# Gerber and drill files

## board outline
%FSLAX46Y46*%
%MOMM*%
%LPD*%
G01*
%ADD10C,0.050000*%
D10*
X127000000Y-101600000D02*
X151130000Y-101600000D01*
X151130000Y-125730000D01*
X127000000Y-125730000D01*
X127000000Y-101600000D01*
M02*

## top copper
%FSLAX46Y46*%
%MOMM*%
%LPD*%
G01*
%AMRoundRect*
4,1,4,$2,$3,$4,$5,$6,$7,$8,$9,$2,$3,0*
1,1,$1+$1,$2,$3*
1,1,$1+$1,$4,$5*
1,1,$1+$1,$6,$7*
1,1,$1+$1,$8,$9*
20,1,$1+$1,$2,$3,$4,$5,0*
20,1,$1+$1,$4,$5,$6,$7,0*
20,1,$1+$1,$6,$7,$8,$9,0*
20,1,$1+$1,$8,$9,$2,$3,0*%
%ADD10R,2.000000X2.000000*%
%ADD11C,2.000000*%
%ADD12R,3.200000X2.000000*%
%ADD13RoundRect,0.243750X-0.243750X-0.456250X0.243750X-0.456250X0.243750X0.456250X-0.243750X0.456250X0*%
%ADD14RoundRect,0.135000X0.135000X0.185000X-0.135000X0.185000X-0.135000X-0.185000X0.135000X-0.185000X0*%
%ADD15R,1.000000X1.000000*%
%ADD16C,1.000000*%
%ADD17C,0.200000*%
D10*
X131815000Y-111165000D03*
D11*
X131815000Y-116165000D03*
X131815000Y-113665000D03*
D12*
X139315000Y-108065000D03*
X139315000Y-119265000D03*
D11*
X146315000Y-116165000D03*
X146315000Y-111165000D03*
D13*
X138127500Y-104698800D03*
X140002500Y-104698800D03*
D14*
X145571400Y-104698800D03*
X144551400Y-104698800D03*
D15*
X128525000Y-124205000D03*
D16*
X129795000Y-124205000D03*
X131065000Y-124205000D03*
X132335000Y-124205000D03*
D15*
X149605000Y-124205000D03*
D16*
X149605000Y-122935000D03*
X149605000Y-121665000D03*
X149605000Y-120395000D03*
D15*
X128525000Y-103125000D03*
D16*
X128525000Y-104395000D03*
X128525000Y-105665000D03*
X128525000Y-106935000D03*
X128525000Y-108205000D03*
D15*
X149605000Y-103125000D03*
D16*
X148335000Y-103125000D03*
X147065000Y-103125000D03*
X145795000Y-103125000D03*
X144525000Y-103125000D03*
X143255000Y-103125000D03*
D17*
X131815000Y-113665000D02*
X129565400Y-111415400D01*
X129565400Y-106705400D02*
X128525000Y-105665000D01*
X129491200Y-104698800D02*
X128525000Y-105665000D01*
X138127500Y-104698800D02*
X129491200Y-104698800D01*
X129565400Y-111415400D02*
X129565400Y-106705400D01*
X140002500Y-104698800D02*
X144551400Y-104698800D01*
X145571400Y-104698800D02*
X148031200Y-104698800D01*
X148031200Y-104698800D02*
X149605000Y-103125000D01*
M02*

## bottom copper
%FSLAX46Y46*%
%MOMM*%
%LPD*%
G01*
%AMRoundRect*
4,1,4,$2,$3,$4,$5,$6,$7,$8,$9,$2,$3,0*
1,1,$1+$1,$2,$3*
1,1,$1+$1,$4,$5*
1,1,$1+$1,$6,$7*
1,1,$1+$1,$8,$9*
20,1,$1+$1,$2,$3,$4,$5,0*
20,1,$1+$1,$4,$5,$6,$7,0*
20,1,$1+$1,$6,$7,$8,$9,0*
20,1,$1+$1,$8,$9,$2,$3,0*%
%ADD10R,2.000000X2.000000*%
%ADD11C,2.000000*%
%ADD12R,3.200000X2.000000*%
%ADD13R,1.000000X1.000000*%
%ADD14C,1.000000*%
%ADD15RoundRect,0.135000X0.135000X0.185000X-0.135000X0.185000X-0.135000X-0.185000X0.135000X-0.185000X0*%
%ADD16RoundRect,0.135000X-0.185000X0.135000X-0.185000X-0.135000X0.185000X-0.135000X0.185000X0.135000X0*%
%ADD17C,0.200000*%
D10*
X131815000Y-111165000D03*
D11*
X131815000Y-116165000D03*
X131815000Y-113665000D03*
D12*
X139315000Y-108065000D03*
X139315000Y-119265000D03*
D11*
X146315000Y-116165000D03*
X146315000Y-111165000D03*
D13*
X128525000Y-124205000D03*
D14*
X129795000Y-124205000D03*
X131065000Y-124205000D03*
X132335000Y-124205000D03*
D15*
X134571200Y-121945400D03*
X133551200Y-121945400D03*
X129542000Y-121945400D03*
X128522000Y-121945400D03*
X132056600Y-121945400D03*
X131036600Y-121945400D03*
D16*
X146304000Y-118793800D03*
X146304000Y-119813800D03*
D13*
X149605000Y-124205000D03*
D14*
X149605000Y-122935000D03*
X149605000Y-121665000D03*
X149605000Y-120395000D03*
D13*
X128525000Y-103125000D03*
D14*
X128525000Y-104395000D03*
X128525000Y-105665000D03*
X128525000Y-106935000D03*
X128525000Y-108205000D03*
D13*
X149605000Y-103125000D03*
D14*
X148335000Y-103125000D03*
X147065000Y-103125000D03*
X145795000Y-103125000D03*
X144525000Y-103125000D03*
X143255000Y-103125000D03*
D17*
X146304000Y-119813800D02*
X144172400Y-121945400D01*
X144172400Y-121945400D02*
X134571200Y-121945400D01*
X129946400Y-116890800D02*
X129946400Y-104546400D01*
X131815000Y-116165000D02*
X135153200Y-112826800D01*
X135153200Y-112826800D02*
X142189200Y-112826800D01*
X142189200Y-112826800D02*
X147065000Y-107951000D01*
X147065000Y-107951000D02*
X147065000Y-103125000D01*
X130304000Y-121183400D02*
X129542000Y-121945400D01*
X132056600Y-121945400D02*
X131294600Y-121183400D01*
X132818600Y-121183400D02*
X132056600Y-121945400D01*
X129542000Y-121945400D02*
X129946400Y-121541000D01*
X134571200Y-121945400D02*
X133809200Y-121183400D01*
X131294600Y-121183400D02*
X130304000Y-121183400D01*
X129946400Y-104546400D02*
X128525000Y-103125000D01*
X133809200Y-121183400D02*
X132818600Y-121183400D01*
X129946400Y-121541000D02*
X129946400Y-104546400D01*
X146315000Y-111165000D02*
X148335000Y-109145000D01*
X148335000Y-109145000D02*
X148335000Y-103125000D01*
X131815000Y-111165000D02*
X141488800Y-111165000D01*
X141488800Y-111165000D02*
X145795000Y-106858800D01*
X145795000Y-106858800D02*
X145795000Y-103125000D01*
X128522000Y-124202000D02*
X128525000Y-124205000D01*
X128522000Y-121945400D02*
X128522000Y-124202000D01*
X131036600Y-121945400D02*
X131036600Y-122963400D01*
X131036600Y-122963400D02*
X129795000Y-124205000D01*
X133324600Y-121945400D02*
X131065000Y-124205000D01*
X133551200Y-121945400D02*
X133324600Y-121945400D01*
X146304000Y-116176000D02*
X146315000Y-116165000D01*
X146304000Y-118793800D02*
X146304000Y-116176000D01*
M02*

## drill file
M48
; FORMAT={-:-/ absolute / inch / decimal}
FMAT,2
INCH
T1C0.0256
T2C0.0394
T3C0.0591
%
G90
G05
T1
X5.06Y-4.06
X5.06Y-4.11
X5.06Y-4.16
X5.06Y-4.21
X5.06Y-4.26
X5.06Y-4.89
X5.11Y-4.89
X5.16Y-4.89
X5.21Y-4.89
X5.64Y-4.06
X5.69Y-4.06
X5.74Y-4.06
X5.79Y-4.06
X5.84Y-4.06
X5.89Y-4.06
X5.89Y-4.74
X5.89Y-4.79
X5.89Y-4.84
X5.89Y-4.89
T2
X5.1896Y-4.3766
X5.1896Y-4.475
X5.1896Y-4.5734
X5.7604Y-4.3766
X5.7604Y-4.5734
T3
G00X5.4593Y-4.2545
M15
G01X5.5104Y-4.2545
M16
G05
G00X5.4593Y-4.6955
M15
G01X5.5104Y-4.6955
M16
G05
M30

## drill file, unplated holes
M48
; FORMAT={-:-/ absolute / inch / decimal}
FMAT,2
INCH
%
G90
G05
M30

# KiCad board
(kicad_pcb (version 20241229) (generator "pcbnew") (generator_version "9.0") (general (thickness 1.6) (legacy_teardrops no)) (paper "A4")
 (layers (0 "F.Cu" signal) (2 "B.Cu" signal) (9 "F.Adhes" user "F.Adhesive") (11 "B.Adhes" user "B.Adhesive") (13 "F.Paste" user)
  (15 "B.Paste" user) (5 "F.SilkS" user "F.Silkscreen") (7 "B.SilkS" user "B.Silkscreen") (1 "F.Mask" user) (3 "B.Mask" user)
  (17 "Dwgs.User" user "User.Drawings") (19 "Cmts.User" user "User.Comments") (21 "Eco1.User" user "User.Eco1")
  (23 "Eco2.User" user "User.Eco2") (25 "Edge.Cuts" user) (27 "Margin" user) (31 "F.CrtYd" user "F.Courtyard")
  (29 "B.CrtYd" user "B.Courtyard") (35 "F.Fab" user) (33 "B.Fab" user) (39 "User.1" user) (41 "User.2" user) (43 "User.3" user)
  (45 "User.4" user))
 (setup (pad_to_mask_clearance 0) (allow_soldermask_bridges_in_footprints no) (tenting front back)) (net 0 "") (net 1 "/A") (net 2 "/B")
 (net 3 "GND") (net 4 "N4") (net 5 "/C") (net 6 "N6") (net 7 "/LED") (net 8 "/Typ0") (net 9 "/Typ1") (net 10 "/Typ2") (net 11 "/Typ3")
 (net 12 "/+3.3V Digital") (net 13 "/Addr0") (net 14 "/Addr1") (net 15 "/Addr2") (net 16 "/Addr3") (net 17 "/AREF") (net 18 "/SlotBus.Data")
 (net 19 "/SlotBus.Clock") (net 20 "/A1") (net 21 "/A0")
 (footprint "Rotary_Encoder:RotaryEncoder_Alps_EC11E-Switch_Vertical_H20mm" (layer "F.Cu") (at 131.815 111.165)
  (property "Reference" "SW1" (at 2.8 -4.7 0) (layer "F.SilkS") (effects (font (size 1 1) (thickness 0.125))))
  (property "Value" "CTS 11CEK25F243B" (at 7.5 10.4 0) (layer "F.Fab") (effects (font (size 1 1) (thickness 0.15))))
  (pad "A" thru_hole rect (at 0 0) (size 2 2) (drill 1) (layers "*.Cu" "*.Mask") (remove_unused_layers no) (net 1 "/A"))
  (pad "B" thru_hole circle (at 0 5) (size 2 2) (drill 1) (layers "*.Cu" "*.Mask") (remove_unused_layers no) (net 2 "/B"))
  (pad "C" thru_hole circle (at 0 2.5) (size 2 2) (drill 1) (layers "*.Cu" "*.Mask") (remove_unused_layers no) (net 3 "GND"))
  (pad "MP" thru_hole rect (at 7.5 -3.1) (size 3.2 2) (drill oval 2.8 1.5) (layers "*.Cu" "*.Mask") (remove_unused_layers no))
  (pad "MP" thru_hole rect (at 7.5 8.1) (size 3.2 2) (drill oval 2.8 1.5) (layers "*.Cu" "*.Mask") (remove_unused_layers no))
  (pad "S1" thru_hole circle (at 14.5 5) (size 2 2) (drill 1) (layers "*.Cu" "*.Mask") (remove_unused_layers no) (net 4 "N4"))
  (pad "S2" thru_hole circle (at 14.5 0) (size 2 2) (drill 1) (layers "*.Cu" "*.Mask") (remove_unused_layers no) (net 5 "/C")))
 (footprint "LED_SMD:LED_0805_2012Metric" (layer "F.Cu") (at 139.065 104.6988)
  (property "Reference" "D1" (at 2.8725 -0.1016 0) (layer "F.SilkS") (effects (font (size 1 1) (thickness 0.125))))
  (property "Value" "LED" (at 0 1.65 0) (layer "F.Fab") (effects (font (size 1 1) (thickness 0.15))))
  (pad "1" smd roundrect (at -0.9375 0) (size 0.975 1.4) (layers "F.Cu" "F.Mask" "F.Paste") (roundrect_rratio 0.25) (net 3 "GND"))
  (pad "2" smd roundrect (at 0.9375 0) (size 0.975 1.4) (layers "F.Cu" "F.Mask" "F.Paste") (roundrect_rratio 0.25) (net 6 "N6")))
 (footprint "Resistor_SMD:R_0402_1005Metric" (layer "F.Cu") (at 145.0614 104.6988 180)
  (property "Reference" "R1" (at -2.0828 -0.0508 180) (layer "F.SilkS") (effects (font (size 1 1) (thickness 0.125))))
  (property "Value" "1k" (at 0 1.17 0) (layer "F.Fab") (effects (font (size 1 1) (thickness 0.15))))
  (pad "1" smd roundrect (at -0.51 0 180) (size 0.54 0.64) (layers "F.Cu" "F.Mask" "F.Paste") (roundrect_rratio 0.25) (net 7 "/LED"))
  (pad "2" smd roundrect (at 0.51 0 180) (size 0.54 0.64) (layers "F.Cu" "F.Mask" "F.Paste") (roundrect_rratio 0.25) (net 6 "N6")))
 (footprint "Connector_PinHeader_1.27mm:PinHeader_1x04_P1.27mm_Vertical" (layer "B.Cu") (at 128.525 124.205 -90)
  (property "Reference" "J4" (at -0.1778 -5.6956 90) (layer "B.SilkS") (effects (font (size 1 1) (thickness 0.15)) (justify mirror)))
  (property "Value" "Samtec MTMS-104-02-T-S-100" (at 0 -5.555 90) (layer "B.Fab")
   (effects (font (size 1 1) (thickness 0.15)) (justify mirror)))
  (pad "1" thru_hole rect (at 0 0 270) (size 1 1) (drill 0.65) (layers "*.Cu" "*.Mask") (remove_unused_layers no) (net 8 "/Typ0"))
  (pad "2" thru_hole circle (at 0 -1.27 270) (size 1 1) (drill 0.65) (layers "*.Cu" "*.Mask") (remove_unused_layers no) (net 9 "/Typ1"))
  (pad "3" thru_hole circle (at 0 -2.54 270) (size 1 1) (drill 0.65) (layers "*.Cu" "*.Mask") (remove_unused_layers no) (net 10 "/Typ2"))
  (pad "4" thru_hole circle (at 0 -3.81 270) (size 1 1) (drill 0.65) (layers "*.Cu" "*.Mask") (remove_unused_layers no) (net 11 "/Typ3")))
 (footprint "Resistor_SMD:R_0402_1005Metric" (layer "B.Cu") (at 134.0612 121.9454 180)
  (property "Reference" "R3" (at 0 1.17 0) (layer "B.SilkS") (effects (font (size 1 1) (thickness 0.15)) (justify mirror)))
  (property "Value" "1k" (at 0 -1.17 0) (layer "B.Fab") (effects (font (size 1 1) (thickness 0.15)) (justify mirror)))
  (pad "1" smd roundrect (at -0.51 0 180) (size 0.54 0.64) (layers "B.Cu" "B.Mask" "B.Paste") (roundrect_rratio 0.25)
   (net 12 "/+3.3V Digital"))
  (pad "2" smd roundrect (at 0.51 0 180) (size 0.54 0.64) (layers "B.Cu" "B.Mask" "B.Paste") (roundrect_rratio 0.25) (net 10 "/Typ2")))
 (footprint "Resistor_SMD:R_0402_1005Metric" (layer "B.Cu") (at 129.032 121.9454 180)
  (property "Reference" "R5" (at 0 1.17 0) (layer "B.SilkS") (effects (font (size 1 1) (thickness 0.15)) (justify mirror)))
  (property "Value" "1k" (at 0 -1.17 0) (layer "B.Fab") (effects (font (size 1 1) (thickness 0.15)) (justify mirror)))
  (pad "1" smd roundrect (at -0.51 0 180) (size 0.54 0.64) (layers "B.Cu" "B.Mask" "B.Paste") (roundrect_rratio 0.25)
   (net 12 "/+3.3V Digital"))
  (pad "2" smd roundrect (at 0.51 0 180) (size 0.54 0.64) (layers "B.Cu" "B.Mask" "B.Paste") (roundrect_rratio 0.25) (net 8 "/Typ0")))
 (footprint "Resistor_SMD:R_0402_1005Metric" (layer "B.Cu") (at 131.5466 121.9454 180)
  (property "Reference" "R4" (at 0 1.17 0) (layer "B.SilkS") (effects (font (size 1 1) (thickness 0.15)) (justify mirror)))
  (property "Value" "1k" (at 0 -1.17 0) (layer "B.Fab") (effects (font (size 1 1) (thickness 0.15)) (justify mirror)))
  (pad "1" smd roundrect (at -0.51 0 180) (size 0.54 0.64) (layers "B.Cu" "B.Mask" "B.Paste") (roundrect_rratio 0.25)
   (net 12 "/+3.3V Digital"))
  (pad "2" smd roundrect (at 0.51 0 180) (size 0.54 0.64) (layers "B.Cu" "B.Mask" "B.Paste") (roundrect_rratio 0.25) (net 9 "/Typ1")))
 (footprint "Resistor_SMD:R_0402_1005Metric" (layer "B.Cu") (at 146.304 119.3038 -90)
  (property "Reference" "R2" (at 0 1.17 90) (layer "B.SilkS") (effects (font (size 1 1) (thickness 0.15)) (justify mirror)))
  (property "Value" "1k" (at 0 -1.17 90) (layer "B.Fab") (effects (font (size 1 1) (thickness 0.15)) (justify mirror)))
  (pad "1" smd roundrect (at -0.51 0 270) (size 0.54 0.64) (layers "B.Cu" "B.Mask" "B.Paste") (roundrect_rratio 0.25) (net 4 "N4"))
  (pad "2" smd roundrect (at 0.51 0 270) (size 0.54 0.64) (layers "B.Cu" "B.Mask" "B.Paste") (roundrect_rratio 0.25)
   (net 12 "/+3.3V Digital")))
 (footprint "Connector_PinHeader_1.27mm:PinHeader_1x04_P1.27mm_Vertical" (layer "B.Cu") (at 149.605 124.205)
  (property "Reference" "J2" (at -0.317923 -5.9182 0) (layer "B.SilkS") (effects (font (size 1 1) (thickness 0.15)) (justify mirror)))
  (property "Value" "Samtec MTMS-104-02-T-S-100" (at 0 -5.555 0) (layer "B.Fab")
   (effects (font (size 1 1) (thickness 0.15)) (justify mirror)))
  (pad "1" thru_hole rect (at 0 0) (size 1 1) (drill 0.65) (layers "*.Cu" "*.Mask") (remove_unused_layers no) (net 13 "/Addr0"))
  (pad "2" thru_hole circle (at 0 -1.27) (size 1 1) (drill 0.65) (layers "*.Cu" "*.Mask") (remove_unused_layers no) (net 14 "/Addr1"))
  (pad "3" thru_hole circle (at 0 -2.54) (size 1 1) (drill 0.65) (layers "*.Cu" "*.Mask") (remove_unused_layers no) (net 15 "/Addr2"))
  (pad "4" thru_hole circle (at 0 -3.81) (size 1 1) (drill 0.65) (layers "*.Cu" "*.Mask") (remove_unused_layers no) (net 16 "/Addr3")))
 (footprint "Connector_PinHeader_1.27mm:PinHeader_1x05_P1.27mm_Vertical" (layer "B.Cu") (at 128.525 103.125 180)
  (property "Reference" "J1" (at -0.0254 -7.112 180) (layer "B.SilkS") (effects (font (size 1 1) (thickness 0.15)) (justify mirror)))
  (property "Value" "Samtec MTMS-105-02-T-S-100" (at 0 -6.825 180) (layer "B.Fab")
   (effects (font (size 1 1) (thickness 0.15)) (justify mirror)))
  (pad "1" thru_hole rect (at 0 0 180) (size 1 1) (drill 0.65) (layers "*.Cu" "*.Mask") (remove_unused_layers no) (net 12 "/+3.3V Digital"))
  (pad "2" thru_hole circle (at 0 -1.27 180) (size 1 1) (drill 0.65) (layers "*.Cu" "*.Mask") (remove_unused_layers no) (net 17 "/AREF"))
  (pad "3" thru_hole circle (at 0 -2.54 180) (size 1 1) (drill 0.65) (layers "*.Cu" "*.Mask") (remove_unused_layers no) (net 3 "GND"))
  (pad "4" thru_hole circle (at 0 -3.81 180) (size 1 1) (drill 0.65) (layers "*.Cu" "*.Mask") (remove_unused_layers no)
   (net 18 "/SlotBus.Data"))
  (pad "5" thru_hole circle (at 0 -5.08 180) (size 1 1) (drill 0.65) (layers "*.Cu" "*.Mask") (remove_unused_layers no)
   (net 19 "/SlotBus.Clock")))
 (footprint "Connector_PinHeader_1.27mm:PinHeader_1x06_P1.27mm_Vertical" (layer "B.Cu") (at 149.605 103.125 90)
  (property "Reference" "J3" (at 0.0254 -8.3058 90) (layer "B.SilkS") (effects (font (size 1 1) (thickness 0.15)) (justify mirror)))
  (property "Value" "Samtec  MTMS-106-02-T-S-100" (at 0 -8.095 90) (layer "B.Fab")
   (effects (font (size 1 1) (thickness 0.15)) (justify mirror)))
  (pad "1" thru_hole rect (at 0 0 90) (size 1 1) (drill 0.65) (layers "*.Cu" "*.Mask") (remove_unused_layers no) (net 7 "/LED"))
  (pad "2" thru_hole circle (at 0 -1.27 90) (size 1 1) (drill 0.65) (layers "*.Cu" "*.Mask") (remove_unused_layers no) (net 5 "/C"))
  (pad "3" thru_hole circle (at 0 -2.54 90) (size 1 1) (drill 0.65) (layers "*.Cu" "*.Mask") (remove_unused_layers no) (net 2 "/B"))
  (pad "4" thru_hole circle (at 0 -3.81 90) (size 1 1) (drill 0.65) (layers "*.Cu" "*.Mask") (remove_unused_layers no) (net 1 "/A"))
  (pad "5" thru_hole circle (at 0 -5.08 90) (size 1 1) (drill 0.65) (layers "*.Cu" "*.Mask") (remove_unused_layers no) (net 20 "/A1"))
  (pad "6" thru_hole circle (at 0 -6.35 90) (size 1 1) (drill 0.65) (layers "*.Cu" "*.Mask") (remove_unused_layers no) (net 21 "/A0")))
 (gr_rect (start 127 101.6) (end 151.13 125.73) (stroke (width 0.05) (type solid)) (fill no) (layer "Edge.Cuts"))
 (segment (start 131.815 113.665) (end 129.5654 111.4154) (width 0.2) (layer "F.Cu") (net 3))
 (segment (start 129.5654 106.7054) (end 128.525 105.665) (width 0.2) (layer "F.Cu") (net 3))
 (segment (start 129.4912 104.6988) (end 128.525 105.665) (width 0.2) (layer "F.Cu") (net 3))
 (segment (start 138.1275 104.6988) (end 129.4912 104.6988) (width 0.2) (layer "F.Cu") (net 3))
 (segment (start 129.5654 111.4154) (end 129.5654 106.7054) (width 0.2) (layer "F.Cu") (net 3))
 (segment (start 140.0025 104.6988) (end 144.5514 104.6988) (width 0.2) (layer "F.Cu") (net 6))
 (segment (start 130.304 121.1834) (end 129.542 121.9454) (width 0.2) (layer "B.Cu") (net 12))
 (segment (start 132.0566 121.9454) (end 131.2946 121.1834) (width 0.2) (layer "B.Cu") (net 12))
 (segment (start 146.304 119.8138) (end 144.1724 121.9454) (width 0.2) (layer "B.Cu") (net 12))
 (segment (start 132.8186 121.1834) (end 132.0566 121.9454) (width 0.2) (layer "B.Cu") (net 12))
 (segment (start 129.542 121.9454) (end 129.9464 121.541) (width 0.2) (layer "B.Cu") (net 12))
 (segment (start 134.5712 121.9454) (end 133.8092 121.1834) (width 0.2) (layer "B.Cu") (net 12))
 (segment (start 131.2946 121.1834) (end 130.304 121.1834) (width 0.2) (layer "B.Cu") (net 12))
 (segment (start 144.1724 121.9454) (end 134.5712 121.9454) (width 0.2) (layer "B.Cu") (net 12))
 (segment (start 129.9464 104.5464) (end 128.525 103.125) (width 0.2) (layer "B.Cu") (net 12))
 (segment (start 129.9464 116.8908) (end 129.9464 104.5464) (width 0.2) (layer "B.Cu") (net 12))
 (segment (start 133.8092 121.1834) (end 132.8186 121.1834) (width 0.2) (layer "B.Cu") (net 12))
 (segment (start 129.9464 121.541) (end 129.9464 104.5464) (width 0.2) (layer "B.Cu") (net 12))
 (segment (start 135.1532 112.8268) (end 142.1892 112.8268) (width 0.2) (layer "B.Cu") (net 2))
 (segment (start 147.065 107.951) (end 147.065 103.125) (width 0.2) (layer "B.Cu") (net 2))
 (segment (start 131.815 116.165) (end 135.1532 112.8268) (width 0.2) (layer "B.Cu") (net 2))
 (segment (start 142.1892 112.8268) (end 147.065 107.951) (width 0.2) (layer "B.Cu") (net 2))
 (segment (start 146.315 111.165) (end 148.335 109.145) (width 0.2) (layer "B.Cu") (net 5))
 (segment (start 148.335 109.145) (end 148.335 103.125) (width 0.2) (layer "B.Cu") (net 5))
 (segment (start 145.5714 104.6988) (end 148.0312 104.6988) (width 0.2) (layer "F.Cu") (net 7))
 (segment (start 148.0312 104.6988) (end 149.605 103.125) (width 0.2) (layer "F.Cu") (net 7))
 (segment (start 131.815 111.165) (end 141.4888 111.165) (width 0.2) (layer "B.Cu") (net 1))
 (segment (start 141.4888 111.165) (end 145.795 106.8588) (width 0.2) (layer "B.Cu") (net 1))
 (segment (start 145.795 106.8588) (end 145.795 103.125) (width 0.2) (layer "B.Cu") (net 1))
 (segment (start 128.522 124.202) (end 128.525 124.205) (width 0.2) (layer "B.Cu") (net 8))
 (segment (start 128.522 121.9454) (end 128.522 124.202) (width 0.2) (layer "B.Cu") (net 8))
 (segment (start 131.0366 121.9454) (end 131.0366 122.9634) (width 0.2) (layer "B.Cu") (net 9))
 (segment (start 131.0366 122.9634) (end 129.795 124.205) (width 0.2) (layer "B.Cu") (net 9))
 (segment (start 133.3246 121.9454) (end 131.065 124.205) (width 0.2) (layer "B.Cu") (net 10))
 (segment (start 133.5512 121.9454) (end 133.3246 121.9454) (width 0.2) (layer "B.Cu") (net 10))
 (segment (start 146.304 116.176) (end 146.315 116.165) (width 0.2) (layer "B.Cu") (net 4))
 (segment (start 146.304 118.7938) (end 146.304 116.176) (width 0.2) (layer "B.Cu") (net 4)))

